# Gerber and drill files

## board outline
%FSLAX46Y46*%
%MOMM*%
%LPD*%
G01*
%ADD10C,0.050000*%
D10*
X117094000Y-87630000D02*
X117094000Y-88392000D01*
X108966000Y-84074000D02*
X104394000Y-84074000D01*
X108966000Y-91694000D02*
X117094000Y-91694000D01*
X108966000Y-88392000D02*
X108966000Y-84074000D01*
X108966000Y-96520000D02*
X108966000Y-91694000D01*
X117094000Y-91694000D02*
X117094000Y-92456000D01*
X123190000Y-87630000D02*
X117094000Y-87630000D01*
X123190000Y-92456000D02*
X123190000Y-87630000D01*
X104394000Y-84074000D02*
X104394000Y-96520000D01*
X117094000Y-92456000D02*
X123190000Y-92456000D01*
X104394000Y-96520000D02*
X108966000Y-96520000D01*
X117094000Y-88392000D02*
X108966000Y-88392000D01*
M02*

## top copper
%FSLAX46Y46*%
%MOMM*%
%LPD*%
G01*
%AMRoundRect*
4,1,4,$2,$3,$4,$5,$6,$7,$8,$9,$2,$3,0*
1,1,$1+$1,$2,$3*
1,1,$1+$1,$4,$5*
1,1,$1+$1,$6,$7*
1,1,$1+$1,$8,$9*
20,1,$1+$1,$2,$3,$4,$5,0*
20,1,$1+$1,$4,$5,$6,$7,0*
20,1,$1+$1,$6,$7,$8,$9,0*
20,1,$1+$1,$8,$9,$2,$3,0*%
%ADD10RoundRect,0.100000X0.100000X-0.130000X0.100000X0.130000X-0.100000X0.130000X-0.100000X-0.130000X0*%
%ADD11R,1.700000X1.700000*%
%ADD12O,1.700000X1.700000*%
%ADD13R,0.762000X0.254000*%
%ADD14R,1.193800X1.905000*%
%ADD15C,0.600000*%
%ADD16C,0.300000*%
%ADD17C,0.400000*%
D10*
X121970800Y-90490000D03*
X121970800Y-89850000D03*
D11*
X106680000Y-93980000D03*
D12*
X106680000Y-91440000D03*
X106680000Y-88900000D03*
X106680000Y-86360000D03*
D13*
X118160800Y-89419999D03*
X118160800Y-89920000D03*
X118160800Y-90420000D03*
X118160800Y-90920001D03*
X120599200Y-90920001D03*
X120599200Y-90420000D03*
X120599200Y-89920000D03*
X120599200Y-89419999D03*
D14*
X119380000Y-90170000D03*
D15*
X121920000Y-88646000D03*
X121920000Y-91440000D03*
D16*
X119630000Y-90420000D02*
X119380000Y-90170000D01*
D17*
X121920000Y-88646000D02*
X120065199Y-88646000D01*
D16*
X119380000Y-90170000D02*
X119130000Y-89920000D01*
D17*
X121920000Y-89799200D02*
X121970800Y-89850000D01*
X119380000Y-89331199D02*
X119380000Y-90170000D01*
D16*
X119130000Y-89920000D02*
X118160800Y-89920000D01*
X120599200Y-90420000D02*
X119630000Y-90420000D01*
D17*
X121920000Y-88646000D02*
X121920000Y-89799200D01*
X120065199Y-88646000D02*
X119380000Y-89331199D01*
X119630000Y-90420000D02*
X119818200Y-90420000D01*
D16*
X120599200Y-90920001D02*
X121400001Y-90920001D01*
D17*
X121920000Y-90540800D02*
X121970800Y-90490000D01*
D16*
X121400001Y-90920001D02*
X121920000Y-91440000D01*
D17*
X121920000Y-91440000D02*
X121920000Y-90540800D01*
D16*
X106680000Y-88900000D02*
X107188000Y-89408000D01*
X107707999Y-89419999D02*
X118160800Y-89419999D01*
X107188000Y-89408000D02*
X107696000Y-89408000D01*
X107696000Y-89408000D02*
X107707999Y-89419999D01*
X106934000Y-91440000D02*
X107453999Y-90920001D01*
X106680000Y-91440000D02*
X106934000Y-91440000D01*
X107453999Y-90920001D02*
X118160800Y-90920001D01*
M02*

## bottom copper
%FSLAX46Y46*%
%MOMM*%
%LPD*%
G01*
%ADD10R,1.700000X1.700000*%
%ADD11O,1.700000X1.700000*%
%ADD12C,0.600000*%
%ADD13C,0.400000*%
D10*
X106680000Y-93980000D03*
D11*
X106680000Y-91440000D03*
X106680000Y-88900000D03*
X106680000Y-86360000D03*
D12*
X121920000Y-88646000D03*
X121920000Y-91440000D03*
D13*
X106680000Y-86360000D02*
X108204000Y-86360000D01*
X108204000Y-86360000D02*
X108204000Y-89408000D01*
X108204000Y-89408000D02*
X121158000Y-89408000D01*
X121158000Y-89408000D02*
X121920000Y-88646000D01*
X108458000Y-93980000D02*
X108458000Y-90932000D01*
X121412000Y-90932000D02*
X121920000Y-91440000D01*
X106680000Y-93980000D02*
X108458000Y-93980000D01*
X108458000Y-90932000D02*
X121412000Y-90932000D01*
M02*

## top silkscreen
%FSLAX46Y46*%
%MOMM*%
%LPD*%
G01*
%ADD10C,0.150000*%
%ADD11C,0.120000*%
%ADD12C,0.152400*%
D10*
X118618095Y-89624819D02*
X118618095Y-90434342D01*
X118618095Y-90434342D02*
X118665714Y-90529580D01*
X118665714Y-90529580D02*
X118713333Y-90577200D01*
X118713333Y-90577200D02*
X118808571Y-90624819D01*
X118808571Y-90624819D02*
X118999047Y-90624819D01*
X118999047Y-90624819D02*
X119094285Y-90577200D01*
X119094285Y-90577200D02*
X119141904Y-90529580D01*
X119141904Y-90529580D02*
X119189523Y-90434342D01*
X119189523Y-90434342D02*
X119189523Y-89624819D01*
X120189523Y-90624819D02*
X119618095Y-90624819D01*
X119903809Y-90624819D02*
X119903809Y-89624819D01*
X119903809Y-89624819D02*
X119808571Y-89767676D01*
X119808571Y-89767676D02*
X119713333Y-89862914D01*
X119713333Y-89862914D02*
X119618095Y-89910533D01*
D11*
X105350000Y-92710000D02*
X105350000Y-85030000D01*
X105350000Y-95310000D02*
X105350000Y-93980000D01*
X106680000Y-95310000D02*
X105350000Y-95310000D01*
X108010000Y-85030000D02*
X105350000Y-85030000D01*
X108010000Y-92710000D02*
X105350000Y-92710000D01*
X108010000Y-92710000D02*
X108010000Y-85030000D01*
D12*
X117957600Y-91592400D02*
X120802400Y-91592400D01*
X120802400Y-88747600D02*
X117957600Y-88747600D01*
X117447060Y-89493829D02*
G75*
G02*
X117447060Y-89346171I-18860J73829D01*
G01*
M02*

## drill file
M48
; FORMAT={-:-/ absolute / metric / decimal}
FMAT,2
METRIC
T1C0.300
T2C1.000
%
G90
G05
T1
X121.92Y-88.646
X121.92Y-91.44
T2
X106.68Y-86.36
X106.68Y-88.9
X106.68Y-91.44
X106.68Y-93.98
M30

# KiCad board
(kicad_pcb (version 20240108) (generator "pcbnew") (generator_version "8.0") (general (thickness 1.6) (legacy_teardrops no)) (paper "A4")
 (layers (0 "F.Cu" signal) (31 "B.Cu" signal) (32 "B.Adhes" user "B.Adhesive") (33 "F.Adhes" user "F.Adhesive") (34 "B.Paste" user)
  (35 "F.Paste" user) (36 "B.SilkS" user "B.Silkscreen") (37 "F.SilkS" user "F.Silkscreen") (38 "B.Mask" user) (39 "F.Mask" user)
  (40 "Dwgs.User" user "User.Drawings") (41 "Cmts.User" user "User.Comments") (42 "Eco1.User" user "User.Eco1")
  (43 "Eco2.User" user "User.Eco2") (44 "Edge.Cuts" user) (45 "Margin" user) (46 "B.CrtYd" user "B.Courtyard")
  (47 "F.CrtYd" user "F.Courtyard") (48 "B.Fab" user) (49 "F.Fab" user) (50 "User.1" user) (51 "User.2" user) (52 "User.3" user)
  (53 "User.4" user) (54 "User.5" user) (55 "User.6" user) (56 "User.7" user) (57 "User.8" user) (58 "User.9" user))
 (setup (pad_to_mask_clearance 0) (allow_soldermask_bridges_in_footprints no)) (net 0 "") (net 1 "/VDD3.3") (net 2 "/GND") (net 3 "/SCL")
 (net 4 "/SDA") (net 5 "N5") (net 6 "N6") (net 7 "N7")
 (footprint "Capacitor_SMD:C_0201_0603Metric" (layer "F.Cu") (at 121.9708 90.17 90)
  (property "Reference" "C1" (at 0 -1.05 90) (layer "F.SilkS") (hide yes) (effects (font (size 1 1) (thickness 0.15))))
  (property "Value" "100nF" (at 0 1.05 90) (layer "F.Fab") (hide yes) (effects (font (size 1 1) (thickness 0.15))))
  (pad "" smd roundrect (at -0.345 0 90) (size 0.318 0.36) (layers "F.Paste") (roundrect_rratio 0.25))
  (pad "" smd roundrect (at 0.345 0 90) (size 0.318 0.36) (layers "F.Paste") (roundrect_rratio 0.25))
  (pad "1" smd roundrect (at -0.32 0 90) (size 0.46 0.4) (layers "F.Cu" "F.Mask") (roundrect_rratio 0.25) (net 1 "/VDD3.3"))
  (pad "2" smd roundrect (at 0.32 0 90) (size 0.46 0.4) (layers "F.Cu" "F.Mask") (roundrect_rratio 0.25) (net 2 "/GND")))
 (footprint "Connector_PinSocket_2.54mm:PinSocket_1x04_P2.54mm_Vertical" (layer "F.Cu") (at 106.68 93.98 180)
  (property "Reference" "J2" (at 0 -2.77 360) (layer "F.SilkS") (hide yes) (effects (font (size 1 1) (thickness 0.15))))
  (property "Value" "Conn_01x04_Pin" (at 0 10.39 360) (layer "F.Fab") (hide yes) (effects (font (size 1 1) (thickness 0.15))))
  (fp_line (start 1.33 1.27) (end 1.33 8.95) (stroke (width 0.12) (type solid)) (layer "F.SilkS"))
  (fp_line (start 1.33 -1.33) (end 1.33 0) (stroke (width 0.12) (type solid)) (layer "F.SilkS"))
  (fp_line (start 0 -1.33) (end 1.33 -1.33) (stroke (width 0.12) (type solid)) (layer "F.SilkS"))
  (fp_line (start -1.33 8.95) (end 1.33 8.95) (stroke (width 0.12) (type solid)) (layer "F.SilkS"))
  (fp_line (start -1.33 1.27) (end 1.33 1.27) (stroke (width 0.12) (type solid)) (layer "F.SilkS"))
  (fp_line (start -1.33 1.27) (end -1.33 8.95) (stroke (width 0.12) (type solid)) (layer "F.SilkS"))
  (pad "1" thru_hole rect (at 0 0 180) (size 1.7 1.7) (drill 1) (layers "*.Cu" "*.Mask") (remove_unused_layers no) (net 1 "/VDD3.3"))
  (pad "2" thru_hole oval (at 0 2.54 180) (size 1.7 1.7) (drill 1) (layers "*.Cu" "*.Mask") (remove_unused_layers no) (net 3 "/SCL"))
  (pad "3" thru_hole oval (at 0 5.08 180) (size 1.7 1.7) (drill 1) (layers "*.Cu" "*.Mask") (remove_unused_layers no) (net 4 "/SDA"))
  (pad "4" thru_hole oval (at 0 7.62 180) (size 1.7 1.7) (drill 1) (layers "*.Cu" "*.Mask") (remove_unused_layers no) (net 2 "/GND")))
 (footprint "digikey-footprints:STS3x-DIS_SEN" (layer "F.Cu") (at 119.38 90.17)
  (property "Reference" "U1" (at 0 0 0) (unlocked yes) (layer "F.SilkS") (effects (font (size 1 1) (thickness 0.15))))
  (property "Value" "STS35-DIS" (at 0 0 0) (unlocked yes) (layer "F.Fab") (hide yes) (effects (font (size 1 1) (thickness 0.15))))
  (fp_line (start -1.4224 1.4224) (end 1.4224 1.4224) (stroke (width 0.1524) (type solid)) (layer "F.SilkS"))
  (fp_line (start 1.4224 -1.4224) (end -1.4224 -1.4224) (stroke (width 0.1524) (type solid)) (layer "F.SilkS"))
  (fp_arc (start -1.93294 -0.676171) (mid -2.028 -0.75) (end -1.93294 -0.823829) (stroke (width 0.1524) (type solid)) (layer "F.SilkS"))
  (pad "1" smd rect (at -1.2192 -0.750001) (size 0.762 0.254) (layers "F.Cu" "F.Paste" "F.Mask") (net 4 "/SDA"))
  (pad "2" smd rect (at -1.2192 -0.25) (size 0.762 0.254) (layers "F.Cu" "F.Paste" "F.Mask") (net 2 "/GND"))
  (pad "3" smd rect (at -1.2192 0.25) (size 0.762 0.254) (layers "F.Cu" "F.Paste" "F.Mask") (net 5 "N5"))
  (pad "4" smd rect (at -1.2192 0.750001) (size 0.762 0.254) (layers "F.Cu" "F.Paste" "F.Mask") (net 3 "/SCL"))
  (pad "5" smd rect (at 1.2192 0.750001) (size 0.762 0.254) (layers "F.Cu" "F.Paste" "F.Mask") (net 1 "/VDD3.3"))
  (pad "6" smd rect (at 1.2192 0.25) (size 0.762 0.254) (layers "F.Cu" "F.Paste" "F.Mask") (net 2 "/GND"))
  (pad "7" smd rect (at 1.2192 -0.25) (size 0.762 0.254) (layers "F.Cu" "F.Paste" "F.Mask") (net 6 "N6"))
  (pad "8" smd rect (at 1.2192 -0.750001) (size 0.762 0.254) (layers "F.Cu" "F.Paste" "F.Mask") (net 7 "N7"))
  (pad "9" smd rect (at 0 0) (size 1.1938 1.905) (layers "F.Cu" "F.Paste" "F.Mask") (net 2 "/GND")))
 (gr_line (start 117.094 87.63) (end 117.094 88.392) (stroke (width 0.05) (type default)) (layer "Edge.Cuts"))
 (gr_line (start 108.966 84.074) (end 104.394 84.074) (stroke (width 0.05) (type default)) (layer "Edge.Cuts"))
 (gr_line (start 108.966 91.694) (end 117.094 91.694) (stroke (width 0.05) (type default)) (layer "Edge.Cuts"))
 (gr_line (start 108.966 88.392) (end 108.966 84.074) (stroke (width 0.05) (type default)) (layer "Edge.Cuts"))
 (gr_line (start 108.966 96.52) (end 108.966 91.694) (stroke (width 0.05) (type default)) (layer "Edge.Cuts"))
 (gr_line (start 117.094 91.694) (end 117.094 92.456) (stroke (width 0.05) (type default)) (layer "Edge.Cuts"))
 (gr_line (start 123.19 87.63) (end 117.094 87.63) (stroke (width 0.05) (type default)) (layer "Edge.Cuts"))
 (gr_line (start 123.19 92.456) (end 123.19 87.63) (stroke (width 0.05) (type default)) (layer "Edge.Cuts"))
 (gr_line (start 104.394 84.074) (end 104.394 96.52) (stroke (width 0.05) (type default)) (layer "Edge.Cuts"))
 (gr_line (start 117.094 92.456) (end 123.19 92.456) (stroke (width 0.05) (type default)) (layer "Edge.Cuts"))
 (gr_line (start 104.394 96.52) (end 108.966 96.52) (stroke (width 0.05) (type default)) (layer "Edge.Cuts"))
 (gr_line (start 117.094 88.392) (end 108.966 88.392) (stroke (width 0.05) (type default)) (layer "Edge.Cuts"))
 (segment (start 119.63 90.42) (end 119.38 90.17) (width 0.3) (layer "F.Cu") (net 2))
 (segment (start 121.92 88.646) (end 120.065199 88.646) (width 0.4) (layer "F.Cu") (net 2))
 (segment (start 119.38 90.17) (end 119.13 89.92) (width 0.3) (layer "F.Cu") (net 2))
 (segment (start 121.92 89.7992) (end 121.9708 89.85) (width 0.4) (layer "F.Cu") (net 2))
 (segment (start 119.38 89.331199) (end 119.38 90.17) (width 0.4) (layer "F.Cu") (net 2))
 (segment (start 119.13 89.92) (end 118.1608 89.92) (width 0.3) (layer "F.Cu") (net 2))
 (segment (start 120.5992 90.42) (end 119.63 90.42) (width 0.3) (layer "F.Cu") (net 2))
 (segment (start 121.92 88.646) (end 121.92 89.7992) (width 0.4) (layer "F.Cu") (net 2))
 (segment (start 120.065199 88.646) (end 119.38 89.331199) (width 0.4) (layer "F.Cu") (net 2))
 (segment (start 119.63 90.42) (end 119.8182 90.42) (width 0.4) (layer "F.Cu") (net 2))
 (via (at 121.92 88.646) (size 0.6) (drill 0.3) (layers "F.Cu" "B.Cu") (free yes) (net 2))
 (segment (start 106.68 86.36) (end 108.204 86.36) (width 0.4) (layer "B.Cu") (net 2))
 (segment (start 108.204 86.36) (end 108.204 89.408) (width 0.4) (layer "B.Cu") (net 2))
 (segment (start 108.204 89.408) (end 121.158 89.408) (width 0.4) (layer "B.Cu") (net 2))
 (segment (start 121.158 89.408) (end 121.92 88.646) (width 0.4) (layer "B.Cu") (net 2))
 (segment (start 120.5992 90.920001) (end 121.400001 90.920001) (width 0.3) (layer "F.Cu") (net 1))
 (segment (start 121.92 90.5408) (end 121.9708 90.49) (width 0.4) (layer "F.Cu") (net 1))
 (segment (start 121.400001 90.920001) (end 121.92 91.44) (width 0.3) (layer "F.Cu") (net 1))
 (segment (start 121.92 91.44) (end 121.92 90.5408) (width 0.4) (layer "F.Cu") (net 1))
 (via (at 121.92 91.44) (size 0.6) (drill 0.3) (layers "F.Cu" "B.Cu") (free yes) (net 1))
 (segment (start 108.458 93.98) (end 108.458 90.932) (width 0.4) (layer "B.Cu") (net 1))
 (segment (start 121.412 90.932) (end 121.92 91.44) (width 0.4) (layer "B.Cu") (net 1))
 (segment (start 106.68 93.98) (end 108.458 93.98) (width 0.4) (layer "B.Cu") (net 1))
 (segment (start 108.458 90.932) (end 121.412 90.932) (width 0.4) (layer "B.Cu") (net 1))
 (segment (start 106.68 88.9) (end 107.188 89.408) (width 0.3) (layer "F.Cu") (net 4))
 (segment (start 107.707999 89.419999) (end 118.1608 89.419999) (width 0.3) (layer "F.Cu") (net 4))
 (segment (start 107.188 89.408) (end 107.696 89.408) (width 0.3) (layer "F.Cu") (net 4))
 (segment (start 107.696 89.408) (end 107.707999 89.419999) (width 0.3) (layer "F.Cu") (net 4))
 (segment (start 106.934 91.44) (end 107.453999 90.920001) (width 0.3) (layer "F.Cu") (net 3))
 (segment (start 106.68 91.44) (end 106.934 91.44) (width 0.3) (layer "F.Cu") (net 3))
 (segment (start 107.453999 90.920001) (end 118.1608 90.920001) (width 0.3) (layer "F.Cu") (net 3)))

